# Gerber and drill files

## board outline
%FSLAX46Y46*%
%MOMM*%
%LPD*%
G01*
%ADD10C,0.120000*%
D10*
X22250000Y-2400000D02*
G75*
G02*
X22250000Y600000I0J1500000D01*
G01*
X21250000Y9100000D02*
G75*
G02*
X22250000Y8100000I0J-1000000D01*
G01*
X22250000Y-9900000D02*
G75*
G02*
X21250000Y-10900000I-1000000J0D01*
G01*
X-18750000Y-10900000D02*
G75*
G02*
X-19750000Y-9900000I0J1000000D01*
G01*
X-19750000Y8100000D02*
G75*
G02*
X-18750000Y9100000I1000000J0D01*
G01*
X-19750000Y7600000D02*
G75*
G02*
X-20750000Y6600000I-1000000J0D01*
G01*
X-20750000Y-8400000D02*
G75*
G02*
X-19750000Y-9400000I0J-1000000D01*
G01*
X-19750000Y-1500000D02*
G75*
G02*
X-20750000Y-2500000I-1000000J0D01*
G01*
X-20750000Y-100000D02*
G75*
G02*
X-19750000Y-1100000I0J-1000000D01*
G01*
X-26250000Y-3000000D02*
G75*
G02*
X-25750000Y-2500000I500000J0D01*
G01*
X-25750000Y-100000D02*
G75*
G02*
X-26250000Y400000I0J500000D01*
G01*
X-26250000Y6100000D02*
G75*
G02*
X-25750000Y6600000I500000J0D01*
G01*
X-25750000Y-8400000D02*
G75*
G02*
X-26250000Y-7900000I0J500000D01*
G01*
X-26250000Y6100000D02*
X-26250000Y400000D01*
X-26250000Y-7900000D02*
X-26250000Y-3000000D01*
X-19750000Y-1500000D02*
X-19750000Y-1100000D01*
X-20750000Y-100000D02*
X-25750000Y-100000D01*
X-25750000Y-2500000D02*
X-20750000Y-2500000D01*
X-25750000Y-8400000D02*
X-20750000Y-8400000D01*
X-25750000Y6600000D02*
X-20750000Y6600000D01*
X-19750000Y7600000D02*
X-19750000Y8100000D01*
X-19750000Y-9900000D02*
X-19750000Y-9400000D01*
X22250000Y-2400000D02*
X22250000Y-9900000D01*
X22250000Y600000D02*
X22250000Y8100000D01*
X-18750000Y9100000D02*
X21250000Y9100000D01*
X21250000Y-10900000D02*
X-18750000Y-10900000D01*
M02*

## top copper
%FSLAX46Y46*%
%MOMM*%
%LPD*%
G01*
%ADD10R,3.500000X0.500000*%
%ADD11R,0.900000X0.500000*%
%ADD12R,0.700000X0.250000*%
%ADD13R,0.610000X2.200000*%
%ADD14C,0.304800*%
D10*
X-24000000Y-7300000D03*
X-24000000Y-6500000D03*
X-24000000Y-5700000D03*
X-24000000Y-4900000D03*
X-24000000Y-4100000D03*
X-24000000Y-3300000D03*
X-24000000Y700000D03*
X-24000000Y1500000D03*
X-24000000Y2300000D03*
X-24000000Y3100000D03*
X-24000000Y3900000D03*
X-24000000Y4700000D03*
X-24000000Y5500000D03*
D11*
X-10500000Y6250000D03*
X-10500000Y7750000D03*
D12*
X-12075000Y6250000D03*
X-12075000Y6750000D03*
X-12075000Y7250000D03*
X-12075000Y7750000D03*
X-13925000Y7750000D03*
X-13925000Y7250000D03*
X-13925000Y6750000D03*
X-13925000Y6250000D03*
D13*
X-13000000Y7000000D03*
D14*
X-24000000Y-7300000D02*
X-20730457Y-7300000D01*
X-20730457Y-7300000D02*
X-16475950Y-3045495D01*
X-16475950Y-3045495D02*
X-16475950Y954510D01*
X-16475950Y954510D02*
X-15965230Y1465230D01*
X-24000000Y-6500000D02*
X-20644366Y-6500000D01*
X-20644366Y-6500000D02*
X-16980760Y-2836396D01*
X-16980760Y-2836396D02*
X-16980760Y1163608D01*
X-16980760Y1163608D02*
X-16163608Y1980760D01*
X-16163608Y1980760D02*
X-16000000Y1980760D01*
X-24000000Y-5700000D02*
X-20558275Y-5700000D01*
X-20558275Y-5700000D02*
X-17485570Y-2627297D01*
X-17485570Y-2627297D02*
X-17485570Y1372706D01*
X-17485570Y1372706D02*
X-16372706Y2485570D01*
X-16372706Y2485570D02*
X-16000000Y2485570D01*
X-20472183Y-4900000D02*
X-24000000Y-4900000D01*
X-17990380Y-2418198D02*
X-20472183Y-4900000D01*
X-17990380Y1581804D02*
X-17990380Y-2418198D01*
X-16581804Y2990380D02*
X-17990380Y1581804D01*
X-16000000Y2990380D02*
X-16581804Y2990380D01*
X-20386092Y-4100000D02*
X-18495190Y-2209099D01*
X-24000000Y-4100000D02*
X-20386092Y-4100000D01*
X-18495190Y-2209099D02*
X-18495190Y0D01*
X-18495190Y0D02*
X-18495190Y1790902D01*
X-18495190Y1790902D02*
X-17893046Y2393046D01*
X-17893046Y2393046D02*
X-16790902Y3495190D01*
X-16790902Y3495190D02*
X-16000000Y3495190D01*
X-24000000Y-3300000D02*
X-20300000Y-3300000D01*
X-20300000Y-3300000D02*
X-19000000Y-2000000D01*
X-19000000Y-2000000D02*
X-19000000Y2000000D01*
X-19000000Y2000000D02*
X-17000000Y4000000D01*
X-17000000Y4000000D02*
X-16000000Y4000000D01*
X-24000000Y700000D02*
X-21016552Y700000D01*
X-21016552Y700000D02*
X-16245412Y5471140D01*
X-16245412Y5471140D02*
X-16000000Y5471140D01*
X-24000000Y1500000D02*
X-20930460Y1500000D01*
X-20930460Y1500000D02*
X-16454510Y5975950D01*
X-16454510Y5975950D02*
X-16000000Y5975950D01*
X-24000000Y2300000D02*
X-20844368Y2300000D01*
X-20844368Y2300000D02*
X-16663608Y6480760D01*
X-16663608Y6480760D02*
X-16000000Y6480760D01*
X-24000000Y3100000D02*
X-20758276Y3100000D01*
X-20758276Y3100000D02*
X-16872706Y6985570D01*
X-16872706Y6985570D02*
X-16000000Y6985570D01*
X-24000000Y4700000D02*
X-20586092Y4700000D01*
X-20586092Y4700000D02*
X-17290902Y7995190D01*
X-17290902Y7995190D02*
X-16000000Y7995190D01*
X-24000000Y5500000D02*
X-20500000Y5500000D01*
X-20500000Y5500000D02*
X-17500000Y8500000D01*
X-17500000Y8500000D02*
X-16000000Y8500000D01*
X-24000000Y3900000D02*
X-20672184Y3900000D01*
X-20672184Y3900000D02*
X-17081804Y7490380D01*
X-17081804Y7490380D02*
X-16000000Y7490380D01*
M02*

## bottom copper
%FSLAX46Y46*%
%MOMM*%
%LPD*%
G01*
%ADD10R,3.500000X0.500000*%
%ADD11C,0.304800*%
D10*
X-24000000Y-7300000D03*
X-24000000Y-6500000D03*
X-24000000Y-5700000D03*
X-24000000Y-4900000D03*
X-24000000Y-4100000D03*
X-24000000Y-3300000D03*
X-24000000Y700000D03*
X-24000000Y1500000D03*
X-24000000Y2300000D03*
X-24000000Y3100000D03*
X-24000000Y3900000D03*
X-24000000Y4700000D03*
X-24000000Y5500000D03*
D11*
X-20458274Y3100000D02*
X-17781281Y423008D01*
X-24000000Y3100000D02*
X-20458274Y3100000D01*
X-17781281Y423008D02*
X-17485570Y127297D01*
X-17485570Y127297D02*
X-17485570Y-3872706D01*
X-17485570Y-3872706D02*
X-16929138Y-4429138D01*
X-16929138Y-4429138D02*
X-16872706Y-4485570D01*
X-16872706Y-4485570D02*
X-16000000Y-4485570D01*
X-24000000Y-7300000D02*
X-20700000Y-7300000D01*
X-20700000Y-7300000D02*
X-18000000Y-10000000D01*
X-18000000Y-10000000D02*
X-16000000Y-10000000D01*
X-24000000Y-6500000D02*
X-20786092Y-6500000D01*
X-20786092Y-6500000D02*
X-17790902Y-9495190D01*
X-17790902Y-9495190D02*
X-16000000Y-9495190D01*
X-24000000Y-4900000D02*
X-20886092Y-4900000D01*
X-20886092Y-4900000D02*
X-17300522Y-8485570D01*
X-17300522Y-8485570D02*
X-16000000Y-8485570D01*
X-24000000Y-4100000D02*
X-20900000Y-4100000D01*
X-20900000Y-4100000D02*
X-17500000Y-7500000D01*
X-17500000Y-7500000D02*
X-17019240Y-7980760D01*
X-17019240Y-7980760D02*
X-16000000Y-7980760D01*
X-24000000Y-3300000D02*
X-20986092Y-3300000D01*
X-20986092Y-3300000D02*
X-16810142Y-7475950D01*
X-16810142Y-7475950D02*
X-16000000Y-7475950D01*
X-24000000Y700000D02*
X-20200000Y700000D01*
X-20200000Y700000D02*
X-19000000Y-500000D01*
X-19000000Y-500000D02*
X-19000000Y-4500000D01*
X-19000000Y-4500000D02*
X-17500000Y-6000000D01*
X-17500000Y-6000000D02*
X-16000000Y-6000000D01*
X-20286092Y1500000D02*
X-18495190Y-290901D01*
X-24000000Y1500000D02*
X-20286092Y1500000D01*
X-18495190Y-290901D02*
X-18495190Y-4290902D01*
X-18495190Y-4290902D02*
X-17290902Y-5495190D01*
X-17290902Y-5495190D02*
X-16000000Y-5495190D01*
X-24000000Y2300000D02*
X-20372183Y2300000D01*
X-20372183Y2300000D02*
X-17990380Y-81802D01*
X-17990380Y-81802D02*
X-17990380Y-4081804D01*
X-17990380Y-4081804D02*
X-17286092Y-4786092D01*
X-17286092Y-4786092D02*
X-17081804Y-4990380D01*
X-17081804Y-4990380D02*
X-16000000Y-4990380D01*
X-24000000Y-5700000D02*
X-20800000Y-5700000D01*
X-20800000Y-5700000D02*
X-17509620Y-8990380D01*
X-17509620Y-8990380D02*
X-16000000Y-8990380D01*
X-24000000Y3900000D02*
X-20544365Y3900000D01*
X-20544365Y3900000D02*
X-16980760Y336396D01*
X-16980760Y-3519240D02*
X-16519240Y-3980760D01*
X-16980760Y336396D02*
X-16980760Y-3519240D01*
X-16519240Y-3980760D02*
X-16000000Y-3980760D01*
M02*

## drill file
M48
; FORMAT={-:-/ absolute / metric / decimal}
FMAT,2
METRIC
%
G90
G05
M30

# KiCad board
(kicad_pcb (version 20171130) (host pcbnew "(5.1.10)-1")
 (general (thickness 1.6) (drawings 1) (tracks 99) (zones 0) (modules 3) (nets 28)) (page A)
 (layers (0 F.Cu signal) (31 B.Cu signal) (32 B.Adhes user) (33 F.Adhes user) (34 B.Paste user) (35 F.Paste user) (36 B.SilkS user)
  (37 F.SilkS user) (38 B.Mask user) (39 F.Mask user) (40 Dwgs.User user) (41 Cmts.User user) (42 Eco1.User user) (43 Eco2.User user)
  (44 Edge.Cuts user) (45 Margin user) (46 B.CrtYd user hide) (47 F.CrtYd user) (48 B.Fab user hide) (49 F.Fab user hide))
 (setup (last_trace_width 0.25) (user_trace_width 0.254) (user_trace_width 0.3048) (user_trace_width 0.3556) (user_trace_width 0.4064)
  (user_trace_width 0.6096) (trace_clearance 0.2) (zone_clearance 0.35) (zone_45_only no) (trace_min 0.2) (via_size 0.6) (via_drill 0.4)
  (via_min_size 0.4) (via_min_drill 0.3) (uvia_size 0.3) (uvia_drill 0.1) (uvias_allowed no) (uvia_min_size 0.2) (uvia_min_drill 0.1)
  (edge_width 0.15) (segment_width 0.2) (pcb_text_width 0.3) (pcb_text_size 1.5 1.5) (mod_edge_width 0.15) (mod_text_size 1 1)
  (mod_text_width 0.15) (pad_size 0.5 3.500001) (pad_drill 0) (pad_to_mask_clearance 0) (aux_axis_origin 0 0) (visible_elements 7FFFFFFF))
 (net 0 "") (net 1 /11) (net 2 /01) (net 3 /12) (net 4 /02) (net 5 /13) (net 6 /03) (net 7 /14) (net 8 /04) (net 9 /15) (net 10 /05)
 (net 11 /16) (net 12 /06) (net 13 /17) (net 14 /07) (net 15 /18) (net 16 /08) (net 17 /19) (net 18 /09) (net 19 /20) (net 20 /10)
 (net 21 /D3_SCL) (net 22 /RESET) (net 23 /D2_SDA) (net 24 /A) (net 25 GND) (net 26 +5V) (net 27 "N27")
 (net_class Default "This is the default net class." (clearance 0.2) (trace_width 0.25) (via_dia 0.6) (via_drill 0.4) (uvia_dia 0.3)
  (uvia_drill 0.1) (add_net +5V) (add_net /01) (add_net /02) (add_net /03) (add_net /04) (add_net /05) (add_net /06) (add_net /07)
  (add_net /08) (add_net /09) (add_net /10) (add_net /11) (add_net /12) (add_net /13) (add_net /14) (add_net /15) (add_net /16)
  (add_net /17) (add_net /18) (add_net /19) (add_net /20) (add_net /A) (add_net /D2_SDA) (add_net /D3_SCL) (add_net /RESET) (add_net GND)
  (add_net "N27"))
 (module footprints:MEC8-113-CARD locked (layer F.Cu) (at -26.25 10.9 90)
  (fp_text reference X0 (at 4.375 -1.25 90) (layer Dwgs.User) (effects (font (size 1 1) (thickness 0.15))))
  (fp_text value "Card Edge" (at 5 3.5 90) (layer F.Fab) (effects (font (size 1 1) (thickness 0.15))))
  (fp_arc (start 10 48.5) (end 11.5 48.5) (angle -180) (layer Edge.Cuts) (width 0.12))
  (fp_arc (start 19 47.5) (end 19 48.5) (angle -90) (layer Edge.Cuts) (width 0.12))
  (fp_arc (start 1 47.5) (end 0 47.5) (angle -90) (layer Edge.Cuts) (width 0.12))
  (fp_arc (start 1 7.5) (end 1 6.5) (angle -90) (layer Edge.Cuts) (width 0.12))
  (fp_arc (start 19 7.5) (end 20 7.5) (angle -90) (layer Edge.Cuts) (width 0.12))
  (fp_arc (start 18.5 5.5) (end 17.5 5.5) (angle -90) (layer Edge.Cuts) (width 0.12))
  (fp_arc (start 1.5 5.5) (end 1.5 6.5) (angle -90) (layer Edge.Cuts) (width 0.12))
  (fp_arc (start 9.4 5.5) (end 8.4 5.5) (angle -90) (layer Edge.Cuts) (width 0.12))
  (fp_arc (start 9.8 5.5) (end 9.8 6.5) (angle -90) (layer Edge.Cuts) (width 0.12))
  (fp_arc (start 7.9 0.5) (end 8.4 0.5) (angle -90) (layer Edge.Cuts) (width 0.12))
  (fp_arc (start 11.3 0.5) (end 11.3 0) (angle -90) (layer Edge.Cuts) (width 0.12))
  (fp_arc (start 17 0.5) (end 17.5 0.5) (angle -90) (layer Edge.Cuts) (width 0.12))
  (fp_arc (start 3 0.5) (end 3 0) (angle -90) (layer Edge.Cuts) (width 0.12))
  (fp_line (start 17 0) (end 11.3 0) (layer Edge.Cuts) (width 0.12))
  (fp_line (start 3 0) (end 7.9 0) (layer Edge.Cuts) (width 0.12))
  (fp_line (start 9.4 6.5) (end 9.8 6.5) (layer Edge.Cuts) (width 0.12))
  (fp_line (start 10.8 5.5) (end 10.8 0.5) (layer Edge.Cuts) (width 0.12))
  (fp_line (start 8.4 0.5) (end 8.4 5.5) (layer Edge.Cuts) (width 0.12))
  (fp_line (start 2.5 0.5) (end 2.5 5.5) (layer Edge.Cuts) (width 0.12))
  (fp_line (start 17.5 0.5) (end 17.5 5.5) (layer Edge.Cuts) (width 0.12))
  (fp_line (start 18.5 6.5) (end 19 6.5) (layer Edge.Cuts) (width 0.12))
  (fp_line (start 1 6.5) (end 1.5 6.5) (layer Edge.Cuts) (width 0.12))
  (fp_line (start 8.5 48.5) (end 1 48.5) (layer Edge.Cuts) (width 0.12))
  (fp_line (start 11.5 48.5) (end 19 48.5) (layer Edge.Cuts) (width 0.12))
  (fp_line (start 20 7.5) (end 20 47.5) (layer Edge.Cuts) (width 0.12))
  (fp_line (start 0 47.5) (end 0 7.5) (layer Edge.Cuts) (width 0.12))
  (pad 14 smd rect (at 3.6 2.25 90) (size 0.5 3.5) (layers F.Cu F.Paste F.Mask) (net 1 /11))
  (pad 1 smd rect (at 3.6 2.25 90) (size 0.5 3.5) (layers B.Cu B.Paste B.Mask) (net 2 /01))
  (pad 15 smd rect (at 4.4 2.25 90) (size 0.5 3.5) (layers F.Cu F.Paste F.Mask) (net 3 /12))
  (pad 2 smd rect (at 4.4 2.25 90) (size 0.5 3.5) (layers B.Cu B.Paste B.Mask) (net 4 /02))
  (pad 16 smd rect (at 5.2 2.25 90) (size 0.5 3.5) (layers F.Cu F.Paste F.Mask) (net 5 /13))
  (pad 3 smd rect (at 5.2 2.25 90) (size 0.5 3.5) (layers B.Cu B.Paste B.Mask) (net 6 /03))
  (pad 17 smd rect (at 6 2.25 90) (size 0.5 3.5) (layers F.Cu F.Paste F.Mask) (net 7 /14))
  (pad 4 smd rect (at 6 2.25 90) (size 0.5 3.5) (layers B.Cu B.Paste B.Mask) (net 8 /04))
  (pad 18 smd rect (at 6.8 2.25 90) (size 0.5 3.5) (layers F.Cu F.Paste F.Mask) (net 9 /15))
  (pad 5 smd rect (at 6.8 2.25 90) (size 0.5 3.5) (layers B.Cu B.Paste B.Mask) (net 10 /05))
  (pad 19 smd rect (at 7.6 2.25 90) (size 0.5 3.5) (layers F.Cu F.Paste F.Mask) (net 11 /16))
  (pad 6 smd rect (at 7.6 2.25 90) (size 0.5 3.5) (layers B.Cu B.Paste B.Mask) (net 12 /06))
  (pad 20 smd rect (at 11.6 2.25 90) (size 0.5 3.5) (layers F.Cu F.Paste F.Mask) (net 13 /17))
  (pad 7 smd rect (at 11.6 2.25 90) (size 0.5 3.5) (layers B.Cu B.Paste B.Mask) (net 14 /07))
  (pad 21 smd rect (at 12.4 2.25 90) (size 0.5 3.5) (layers F.Cu F.Paste F.Mask) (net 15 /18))
  (pad 8 smd rect (at 12.4 2.25 90) (size 0.5 3.5) (layers B.Cu B.Paste B.Mask) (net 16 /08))
  (pad 22 smd rect (at 13.2 2.25 90) (size 0.5 3.5) (layers F.Cu F.Paste F.Mask) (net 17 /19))
  (pad 9 smd rect (at 13.2 2.25 90) (size 0.5 3.5) (layers B.Cu B.Paste B.Mask) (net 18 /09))
  (pad 23 smd rect (at 14 2.25 90) (size 0.5 3.5) (layers F.Cu F.Paste F.Mask) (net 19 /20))
  (pad 10 smd rect (at 14 2.25 90) (size 0.5 3.5) (layers B.Cu B.Paste B.Mask) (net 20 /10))
  (pad 24 smd rect (at 14.8 2.25 90) (size 0.5 3.5) (layers F.Cu F.Paste F.Mask) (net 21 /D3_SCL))
  (pad 11 smd rect (at 14.8 2.25 90) (size 0.5 3.5) (layers B.Cu B.Paste B.Mask) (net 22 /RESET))
  (pad 25 smd rect (at 15.6 2.25 90) (size 0.5 3.5) (layers F.Cu F.Paste F.Mask) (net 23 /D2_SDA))
  (pad 12 smd rect (at 15.6 2.25 90) (size 0.5 3.5) (layers B.Cu B.Paste B.Mask) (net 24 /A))
  (pad 26 smd rect (at 16.4 2.25 90) (size 0.5 3.5) (layers F.Cu F.Paste F.Mask) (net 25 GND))
  (pad 13 smd rect (at 16.4 2.25 90) (size 0.5 3.5) (layers B.Cu B.Paste B.Mask) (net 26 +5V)))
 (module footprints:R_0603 (layer F.Cu) (at -10.5 -7 90)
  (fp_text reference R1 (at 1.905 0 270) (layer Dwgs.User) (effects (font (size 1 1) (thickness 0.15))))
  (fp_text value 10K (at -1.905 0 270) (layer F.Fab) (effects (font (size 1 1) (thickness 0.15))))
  (pad 1 smd rect (at -0.75 0 90) (size 0.5 0.9) (layers F.Cu F.Paste F.Mask) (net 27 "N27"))
  (pad 2 smd rect (at 0.75 0 90) (size 0.5 0.9) (layers F.Cu F.Paste F.Mask) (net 24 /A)))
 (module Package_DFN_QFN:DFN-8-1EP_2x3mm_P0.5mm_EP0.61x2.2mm (layer F.Cu) (at -13 -7 180)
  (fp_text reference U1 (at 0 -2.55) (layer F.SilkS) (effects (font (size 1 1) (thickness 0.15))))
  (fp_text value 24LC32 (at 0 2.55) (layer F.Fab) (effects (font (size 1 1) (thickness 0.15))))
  (pad 1 smd rect (at -0.925 -0.75 180) (size 0.7 0.25) (layers F.Cu F.Paste F.Mask) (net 27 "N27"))
  (pad 2 smd rect (at -0.925 -0.25 180) (size 0.7 0.25) (layers F.Cu F.Paste F.Mask) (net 25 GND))
  (pad 3 smd rect (at -0.925 0.25 180) (size 0.7 0.25) (layers F.Cu F.Paste F.Mask) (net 25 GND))
  (pad 4 smd rect (at -0.925 0.75 180) (size 0.7 0.25) (layers F.Cu F.Paste F.Mask) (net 25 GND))
  (pad 5 smd rect (at 0.925 0.75 180) (size 0.7 0.25) (layers F.Cu F.Paste F.Mask) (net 23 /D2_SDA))
  (pad 6 smd rect (at 0.925 0.25 180) (size 0.7 0.25) (layers F.Cu F.Paste F.Mask) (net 21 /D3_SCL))
  (pad 7 smd rect (at 0.925 -0.25 180) (size 0.7 0.25) (layers F.Cu F.Paste F.Mask))
  (pad 8 smd rect (at 0.925 -0.75 180) (size 0.7 0.25) (layers F.Cu F.Paste F.Mask) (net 26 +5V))
  (pad 9 smd rect (at 0 0 180) (size 0.61 2.2) (layers F.Cu F.Mask))
  (pad "" smd rect (at 0 -0.734 180) (size 0.5 0.59) (layers F.Paste))
  (pad "" smd rect (at 0 0 180) (size 0.5 0.59) (layers F.Paste))
  (pad "" smd rect (at 0 0.734 180) (size 0.5 0.59) (layers F.Paste)))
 (segment (start -20.458274 -3.1) (end -17.781281 -0.423008) (width 0.3048) (layer B.Cu) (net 20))
 (segment (start -24 -3.1) (end -20.458274 -3.1) (width 0.3048) (layer B.Cu) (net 20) (status 10))
 (segment (start -17.781281 -0.423008) (end -17.48557 -0.127297) (width 0.3048) (layer B.Cu) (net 20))
 (segment (start -17.48557 -0.127297) (end -17.48557 3.872706) (width 0.3048) (layer B.Cu) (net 20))
 (segment (start -17.48557 3.872706) (end -16.929138 4.429138) (width 0.3048) (layer B.Cu) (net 20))
 (segment (start -16.929138 4.429138) (end -16.872706 4.48557) (width 0.3048) (layer B.Cu) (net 20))
 (segment (start -16.872706 4.48557) (end -16 4.48557) (width 0.3048) (layer B.Cu) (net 20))
 (segment (start -24 7.3) (end -20.7 7.3) (width 0.3048) (layer B.Cu) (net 2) (status 10))
 (segment (start -20.7 7.3) (end -18 10) (width 0.3048) (layer B.Cu) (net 2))
 (segment (start -18 10) (end -16 10) (width 0.3048) (layer B.Cu) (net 2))
 (segment (start -24 6.5) (end -20.786092 6.5) (width 0.3048) (layer B.Cu) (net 4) (status 10))
 (segment (start -20.786092 6.5) (end -17.790902 9.49519) (width 0.3048) (layer B.Cu) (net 4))
 (segment (start -17.790902 9.49519) (end -16 9.49519) (width 0.3048) (layer B.Cu) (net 4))
 (segment (start -24 4.9) (end -20.886092 4.9) (width 0.3048) (layer B.Cu) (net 8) (status 10))
 (segment (start -20.886092 4.9) (end -17.300522 8.48557) (width 0.3048) (layer B.Cu) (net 8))
 (segment (start -17.300522 8.48557) (end -16 8.48557) (width 0.3048) (layer B.Cu) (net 8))
 (segment (start -24 4.1) (end -20.9 4.1) (width 0.3048) (layer B.Cu) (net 10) (status 10))
 (segment (start -20.9 4.1) (end -17.5 7.5) (width 0.3048) (layer B.Cu) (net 10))
 (segment (start -17.5 7.5) (end -17.01924 7.98076) (width 0.3048) (layer B.Cu) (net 10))
 (segment (start -17.01924 7.98076) (end -16 7.98076) (width 0.3048) (layer B.Cu) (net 10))
 (segment (start -24 3.3) (end -20.986092 3.3) (width 0.3048) (layer B.Cu) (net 12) (status 10))
 (segment (start -20.986092 3.3) (end -16.810142 7.47595) (width 0.3048) (layer B.Cu) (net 12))
 (segment (start -16.810142 7.47595) (end -16 7.47595) (width 0.3048) (layer B.Cu) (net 12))
 (segment (start -24 -0.7) (end -20.2 -0.7) (width 0.3048) (layer B.Cu) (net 14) (status 10))
 (segment (start -20.2 -0.7) (end -19 0.5) (width 0.3048) (layer B.Cu) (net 14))
 (segment (start -19 0.5) (end -19 4.5) (width 0.3048) (layer B.Cu) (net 14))
 (segment (start -19 4.5) (end -17.5 6) (width 0.3048) (layer B.Cu) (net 14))
 (segment (start -17.5 6) (end -16 6) (width 0.3048) (layer B.Cu) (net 14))
 (segment (start -20.286092 -1.5) (end -18.49519 0.290901) (width 0.3048) (layer B.Cu) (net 16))
 (segment (start -24 -1.5) (end -20.286092 -1.5) (width 0.3048) (layer B.Cu) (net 16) (status 10))
 (segment (start -18.49519 0.290901) (end -18.49519 4.290902) (width 0.3048) (layer B.Cu) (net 16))
 (segment (start -18.49519 4.290902) (end -17.290902 5.49519) (width 0.3048) (layer B.Cu) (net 16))
 (segment (start -17.290902 5.49519) (end -16 5.49519) (width 0.3048) (layer B.Cu) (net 16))
 (segment (start -24 -2.3) (end -20.372183 -2.3) (width 0.3048) (layer B.Cu) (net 18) (status 10))
 (segment (start -20.372183 -2.3) (end -17.99038 0.081802) (width 0.3048) (layer B.Cu) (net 18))
 (segment (start -17.99038 0.081802) (end -17.99038 4.081804) (width 0.3048) (layer B.Cu) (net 18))
 (segment (start -17.99038 4.081804) (end -17.286092 4.786092) (width 0.3048) (layer B.Cu) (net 18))
 (segment (start -17.286092 4.786092) (end -17.081804 4.99038) (width 0.3048) (layer B.Cu) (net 18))
 (segment (start -17.081804 4.99038) (end -16 4.99038) (width 0.3048) (layer B.Cu) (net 18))
 (segment (start -24 7.3) (end -20.730457 7.3) (width 0.3048) (layer F.Cu) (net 1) (status 10))
 (segment (start -20.730457 7.3) (end -16.47595 3.045495) (width 0.3048) (layer F.Cu) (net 1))
 (segment (start -16.47595 3.045495) (end -16.47595 -0.95451) (width 0.3048) (layer F.Cu) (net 1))
 (segment (start -16.47595 -0.95451) (end -15.96523 -1.46523) (width 0.3048) (layer F.Cu) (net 1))
 (segment (start -24 6.5) (end -20.644366 6.5) (width 0.3048) (layer F.Cu) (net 3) (status 10))
 (segment (start -20.644366 6.5) (end -16.98076 2.836396) (width 0.3048) (layer F.Cu) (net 3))
 (segment (start -16.98076 2.836396) (end -16.98076 -1.163608) (width 0.3048) (layer F.Cu) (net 3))
 (segment (start -16.98076 -1.163608) (end -16.163608 -1.98076) (width 0.3048) (layer F.Cu) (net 3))
 (segment (start -16.163608 -1.98076) (end -16 -1.98076) (width 0.3048) (layer F.Cu) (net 3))
 (segment (start -24 5.7) (end -20.558275 5.7) (width 0.3048) (layer F.Cu) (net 5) (status 10))
 (segment (start -20.558275 5.7) (end -17.48557 2.627297) (width 0.3048) (layer F.Cu) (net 5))
 (segment (start -17.48557 2.627297) (end -17.48557 -1.372706) (width 0.3048) (layer F.Cu) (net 5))
 (segment (start -17.48557 -1.372706) (end -16.372706 -2.48557) (width 0.3048) (layer F.Cu) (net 5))
 (segment (start -16.372706 -2.48557) (end -16 -2.48557) (width 0.3048) (layer F.Cu) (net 5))
 (segment (start -20.472183 4.9) (end -24 4.9) (width 0.3048) (layer F.Cu) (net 7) (status 20))
 (segment (start -17.99038 2.418198) (end -20.472183 4.9) (width 0.3048) (layer F.Cu) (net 7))
 (segment (start -17.99038 -1.581804) (end -17.99038 2.418198) (width 0.3048) (layer F.Cu) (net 7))
 (segment (start -16.581804 -2.99038) (end -17.99038 -1.581804) (width 0.3048) (layer F.Cu) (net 7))
 (segment (start -16 -2.99038) (end -16.581804 -2.99038) (width 0.3048) (layer F.Cu) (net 7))
 (segment (start -20.386092 4.1) (end -18.49519 2.209099) (width 0.3048) (layer F.Cu) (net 9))
 (segment (start -24 4.1) (end -20.386092 4.1) (width 0.3048) (layer F.Cu) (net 9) (status 10))
 (segment (start -18.49519 2.209099) (end -18.49519 0) (width 0.3048) (layer F.Cu) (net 9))
 (segment (start -18.49519 0) (end -18.49519 -1.790902) (width 0.3048) (layer F.Cu) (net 9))
 (segment (start -18.49519 -1.790902) (end -17.893046 -2.393046) (width 0.3048) (layer F.Cu) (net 9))
 (segment (start -17.893046 -2.393046) (end -16.790902 -3.49519) (width 0.3048) (layer F.Cu) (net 9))
 (segment (start -16.790902 -3.49519) (end -16 -3.49519) (width 0.3048) (layer F.Cu) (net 9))
 (segment (start -24 3.3) (end -20.3 3.3) (width 0.3048) (layer F.Cu) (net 11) (status 10))
 (segment (start -20.3 3.3) (end -19 2) (width 0.3048) (layer F.Cu) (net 11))
 (segment (start -19 2) (end -19 -2) (width 0.3048) (layer F.Cu) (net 11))
 (segment (start -19 -2) (end -17 -4) (width 0.3048) (layer F.Cu) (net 11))
 (segment (start -17 -4) (end -16 -4) (width 0.3048) (layer F.Cu) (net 11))
 (segment (start -24 -0.7) (end -21.016552 -0.7) (width 0.3048) (layer F.Cu) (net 13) (status 10))
 (segment (start -21.016552 -0.7) (end -16.245412 -5.47114) (width 0.3048) (layer F.Cu) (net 13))
 (segment (start -16.245412 -5.47114) (end -16 -5.47114) (width 0.3048) (layer F.Cu) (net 13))
 (segment (start -24 -1.5) (end -20.93046 -1.5) (width 0.3048) (layer F.Cu) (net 15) (status 10))
 (segment (start -20.93046 -1.5) (end -16.45451 -5.97595) (width 0.3048) (layer F.Cu) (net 15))
 (segment (start -16.45451 -5.97595) (end -16 -5.97595) (width 0.3048) (layer F.Cu) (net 15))
 (segment (start -24 -2.3) (end -20.844368 -2.3) (width 0.3048) (layer F.Cu) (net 17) (status 10))
 (segment (start -20.844368 -2.3) (end -16.663608 -6.48076) (width 0.3048) (layer F.Cu) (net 17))
 (segment (start -16.663608 -6.48076) (end -16 -6.48076) (width 0.3048) (layer F.Cu) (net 17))
 (segment (start -24 -3.1) (end -20.758276 -3.1) (width 0.3048) (layer F.Cu) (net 19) (status 10))
 (segment (start -20.758276 -3.1) (end -16.872706 -6.98557) (width 0.3048) (layer F.Cu) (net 19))
 (segment (start -16.872706 -6.98557) (end -16 -6.98557) (width 0.3048) (layer F.Cu) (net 19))
 (segment (start -24 5.7) (end -20.8 5.7) (width 0.3048) (layer B.Cu) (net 6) (status 10))
 (segment (start -20.8 5.7) (end -17.50962 8.99038) (width 0.3048) (layer B.Cu) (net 6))
 (segment (start -17.50962 8.99038) (end -16 8.99038) (width 0.3048) (layer B.Cu) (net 6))
 (segment (start -24 -4.7) (end -20.586092 -4.7) (width 0.3048) (layer F.Cu) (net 23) (status 10))
 (segment (start -20.586092 -4.7) (end -17.290902 -7.99519) (width 0.3048) (layer F.Cu) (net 23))
 (segment (start -17.290902 -7.99519) (end -16 -7.99519) (width 0.3048) (layer F.Cu) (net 23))
 (segment (start -24 -5.5) (end -20.5 -5.5) (width 0.3048) (layer F.Cu) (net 25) (status 10))
 (segment (start -20.5 -5.5) (end -17.5 -8.5) (width 0.3048) (layer F.Cu) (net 25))
 (segment (start -17.5 -8.5) (end -16 -8.5) (width 0.3048) (layer F.Cu) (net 25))
 (segment (start -24 -3.9) (end -20.672184 -3.9) (width 0.3048) (layer F.Cu) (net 21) (status 10))
 (segment (start -20.672184 -3.9) (end -17.081804 -7.49038) (width 0.3048) (layer F.Cu) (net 21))
 (segment (start -17.081804 -7.49038) (end -16 -7.49038) (width 0.3048) (layer F.Cu) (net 21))
 (segment (start -24 -3.9) (end -20.544365 -3.9) (width 0.3048) (layer B.Cu) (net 22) (status 10))
 (segment (start -20.544365 -3.9) (end -16.98076 -0.336396) (width 0.3048) (layer B.Cu) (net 22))
 (segment (start -16.98076 3.51924) (end -16.51924 3.98076) (width 0.3048) (layer B.Cu) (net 22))
 (segment (start -16.98076 -0.336396) (end -16.98076 3.51924) (width 0.3048) (layer B.Cu) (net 22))
 (segment (start -16.51924 3.98076) (end -16 3.98076) (width 0.3048) (layer B.Cu) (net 22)))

